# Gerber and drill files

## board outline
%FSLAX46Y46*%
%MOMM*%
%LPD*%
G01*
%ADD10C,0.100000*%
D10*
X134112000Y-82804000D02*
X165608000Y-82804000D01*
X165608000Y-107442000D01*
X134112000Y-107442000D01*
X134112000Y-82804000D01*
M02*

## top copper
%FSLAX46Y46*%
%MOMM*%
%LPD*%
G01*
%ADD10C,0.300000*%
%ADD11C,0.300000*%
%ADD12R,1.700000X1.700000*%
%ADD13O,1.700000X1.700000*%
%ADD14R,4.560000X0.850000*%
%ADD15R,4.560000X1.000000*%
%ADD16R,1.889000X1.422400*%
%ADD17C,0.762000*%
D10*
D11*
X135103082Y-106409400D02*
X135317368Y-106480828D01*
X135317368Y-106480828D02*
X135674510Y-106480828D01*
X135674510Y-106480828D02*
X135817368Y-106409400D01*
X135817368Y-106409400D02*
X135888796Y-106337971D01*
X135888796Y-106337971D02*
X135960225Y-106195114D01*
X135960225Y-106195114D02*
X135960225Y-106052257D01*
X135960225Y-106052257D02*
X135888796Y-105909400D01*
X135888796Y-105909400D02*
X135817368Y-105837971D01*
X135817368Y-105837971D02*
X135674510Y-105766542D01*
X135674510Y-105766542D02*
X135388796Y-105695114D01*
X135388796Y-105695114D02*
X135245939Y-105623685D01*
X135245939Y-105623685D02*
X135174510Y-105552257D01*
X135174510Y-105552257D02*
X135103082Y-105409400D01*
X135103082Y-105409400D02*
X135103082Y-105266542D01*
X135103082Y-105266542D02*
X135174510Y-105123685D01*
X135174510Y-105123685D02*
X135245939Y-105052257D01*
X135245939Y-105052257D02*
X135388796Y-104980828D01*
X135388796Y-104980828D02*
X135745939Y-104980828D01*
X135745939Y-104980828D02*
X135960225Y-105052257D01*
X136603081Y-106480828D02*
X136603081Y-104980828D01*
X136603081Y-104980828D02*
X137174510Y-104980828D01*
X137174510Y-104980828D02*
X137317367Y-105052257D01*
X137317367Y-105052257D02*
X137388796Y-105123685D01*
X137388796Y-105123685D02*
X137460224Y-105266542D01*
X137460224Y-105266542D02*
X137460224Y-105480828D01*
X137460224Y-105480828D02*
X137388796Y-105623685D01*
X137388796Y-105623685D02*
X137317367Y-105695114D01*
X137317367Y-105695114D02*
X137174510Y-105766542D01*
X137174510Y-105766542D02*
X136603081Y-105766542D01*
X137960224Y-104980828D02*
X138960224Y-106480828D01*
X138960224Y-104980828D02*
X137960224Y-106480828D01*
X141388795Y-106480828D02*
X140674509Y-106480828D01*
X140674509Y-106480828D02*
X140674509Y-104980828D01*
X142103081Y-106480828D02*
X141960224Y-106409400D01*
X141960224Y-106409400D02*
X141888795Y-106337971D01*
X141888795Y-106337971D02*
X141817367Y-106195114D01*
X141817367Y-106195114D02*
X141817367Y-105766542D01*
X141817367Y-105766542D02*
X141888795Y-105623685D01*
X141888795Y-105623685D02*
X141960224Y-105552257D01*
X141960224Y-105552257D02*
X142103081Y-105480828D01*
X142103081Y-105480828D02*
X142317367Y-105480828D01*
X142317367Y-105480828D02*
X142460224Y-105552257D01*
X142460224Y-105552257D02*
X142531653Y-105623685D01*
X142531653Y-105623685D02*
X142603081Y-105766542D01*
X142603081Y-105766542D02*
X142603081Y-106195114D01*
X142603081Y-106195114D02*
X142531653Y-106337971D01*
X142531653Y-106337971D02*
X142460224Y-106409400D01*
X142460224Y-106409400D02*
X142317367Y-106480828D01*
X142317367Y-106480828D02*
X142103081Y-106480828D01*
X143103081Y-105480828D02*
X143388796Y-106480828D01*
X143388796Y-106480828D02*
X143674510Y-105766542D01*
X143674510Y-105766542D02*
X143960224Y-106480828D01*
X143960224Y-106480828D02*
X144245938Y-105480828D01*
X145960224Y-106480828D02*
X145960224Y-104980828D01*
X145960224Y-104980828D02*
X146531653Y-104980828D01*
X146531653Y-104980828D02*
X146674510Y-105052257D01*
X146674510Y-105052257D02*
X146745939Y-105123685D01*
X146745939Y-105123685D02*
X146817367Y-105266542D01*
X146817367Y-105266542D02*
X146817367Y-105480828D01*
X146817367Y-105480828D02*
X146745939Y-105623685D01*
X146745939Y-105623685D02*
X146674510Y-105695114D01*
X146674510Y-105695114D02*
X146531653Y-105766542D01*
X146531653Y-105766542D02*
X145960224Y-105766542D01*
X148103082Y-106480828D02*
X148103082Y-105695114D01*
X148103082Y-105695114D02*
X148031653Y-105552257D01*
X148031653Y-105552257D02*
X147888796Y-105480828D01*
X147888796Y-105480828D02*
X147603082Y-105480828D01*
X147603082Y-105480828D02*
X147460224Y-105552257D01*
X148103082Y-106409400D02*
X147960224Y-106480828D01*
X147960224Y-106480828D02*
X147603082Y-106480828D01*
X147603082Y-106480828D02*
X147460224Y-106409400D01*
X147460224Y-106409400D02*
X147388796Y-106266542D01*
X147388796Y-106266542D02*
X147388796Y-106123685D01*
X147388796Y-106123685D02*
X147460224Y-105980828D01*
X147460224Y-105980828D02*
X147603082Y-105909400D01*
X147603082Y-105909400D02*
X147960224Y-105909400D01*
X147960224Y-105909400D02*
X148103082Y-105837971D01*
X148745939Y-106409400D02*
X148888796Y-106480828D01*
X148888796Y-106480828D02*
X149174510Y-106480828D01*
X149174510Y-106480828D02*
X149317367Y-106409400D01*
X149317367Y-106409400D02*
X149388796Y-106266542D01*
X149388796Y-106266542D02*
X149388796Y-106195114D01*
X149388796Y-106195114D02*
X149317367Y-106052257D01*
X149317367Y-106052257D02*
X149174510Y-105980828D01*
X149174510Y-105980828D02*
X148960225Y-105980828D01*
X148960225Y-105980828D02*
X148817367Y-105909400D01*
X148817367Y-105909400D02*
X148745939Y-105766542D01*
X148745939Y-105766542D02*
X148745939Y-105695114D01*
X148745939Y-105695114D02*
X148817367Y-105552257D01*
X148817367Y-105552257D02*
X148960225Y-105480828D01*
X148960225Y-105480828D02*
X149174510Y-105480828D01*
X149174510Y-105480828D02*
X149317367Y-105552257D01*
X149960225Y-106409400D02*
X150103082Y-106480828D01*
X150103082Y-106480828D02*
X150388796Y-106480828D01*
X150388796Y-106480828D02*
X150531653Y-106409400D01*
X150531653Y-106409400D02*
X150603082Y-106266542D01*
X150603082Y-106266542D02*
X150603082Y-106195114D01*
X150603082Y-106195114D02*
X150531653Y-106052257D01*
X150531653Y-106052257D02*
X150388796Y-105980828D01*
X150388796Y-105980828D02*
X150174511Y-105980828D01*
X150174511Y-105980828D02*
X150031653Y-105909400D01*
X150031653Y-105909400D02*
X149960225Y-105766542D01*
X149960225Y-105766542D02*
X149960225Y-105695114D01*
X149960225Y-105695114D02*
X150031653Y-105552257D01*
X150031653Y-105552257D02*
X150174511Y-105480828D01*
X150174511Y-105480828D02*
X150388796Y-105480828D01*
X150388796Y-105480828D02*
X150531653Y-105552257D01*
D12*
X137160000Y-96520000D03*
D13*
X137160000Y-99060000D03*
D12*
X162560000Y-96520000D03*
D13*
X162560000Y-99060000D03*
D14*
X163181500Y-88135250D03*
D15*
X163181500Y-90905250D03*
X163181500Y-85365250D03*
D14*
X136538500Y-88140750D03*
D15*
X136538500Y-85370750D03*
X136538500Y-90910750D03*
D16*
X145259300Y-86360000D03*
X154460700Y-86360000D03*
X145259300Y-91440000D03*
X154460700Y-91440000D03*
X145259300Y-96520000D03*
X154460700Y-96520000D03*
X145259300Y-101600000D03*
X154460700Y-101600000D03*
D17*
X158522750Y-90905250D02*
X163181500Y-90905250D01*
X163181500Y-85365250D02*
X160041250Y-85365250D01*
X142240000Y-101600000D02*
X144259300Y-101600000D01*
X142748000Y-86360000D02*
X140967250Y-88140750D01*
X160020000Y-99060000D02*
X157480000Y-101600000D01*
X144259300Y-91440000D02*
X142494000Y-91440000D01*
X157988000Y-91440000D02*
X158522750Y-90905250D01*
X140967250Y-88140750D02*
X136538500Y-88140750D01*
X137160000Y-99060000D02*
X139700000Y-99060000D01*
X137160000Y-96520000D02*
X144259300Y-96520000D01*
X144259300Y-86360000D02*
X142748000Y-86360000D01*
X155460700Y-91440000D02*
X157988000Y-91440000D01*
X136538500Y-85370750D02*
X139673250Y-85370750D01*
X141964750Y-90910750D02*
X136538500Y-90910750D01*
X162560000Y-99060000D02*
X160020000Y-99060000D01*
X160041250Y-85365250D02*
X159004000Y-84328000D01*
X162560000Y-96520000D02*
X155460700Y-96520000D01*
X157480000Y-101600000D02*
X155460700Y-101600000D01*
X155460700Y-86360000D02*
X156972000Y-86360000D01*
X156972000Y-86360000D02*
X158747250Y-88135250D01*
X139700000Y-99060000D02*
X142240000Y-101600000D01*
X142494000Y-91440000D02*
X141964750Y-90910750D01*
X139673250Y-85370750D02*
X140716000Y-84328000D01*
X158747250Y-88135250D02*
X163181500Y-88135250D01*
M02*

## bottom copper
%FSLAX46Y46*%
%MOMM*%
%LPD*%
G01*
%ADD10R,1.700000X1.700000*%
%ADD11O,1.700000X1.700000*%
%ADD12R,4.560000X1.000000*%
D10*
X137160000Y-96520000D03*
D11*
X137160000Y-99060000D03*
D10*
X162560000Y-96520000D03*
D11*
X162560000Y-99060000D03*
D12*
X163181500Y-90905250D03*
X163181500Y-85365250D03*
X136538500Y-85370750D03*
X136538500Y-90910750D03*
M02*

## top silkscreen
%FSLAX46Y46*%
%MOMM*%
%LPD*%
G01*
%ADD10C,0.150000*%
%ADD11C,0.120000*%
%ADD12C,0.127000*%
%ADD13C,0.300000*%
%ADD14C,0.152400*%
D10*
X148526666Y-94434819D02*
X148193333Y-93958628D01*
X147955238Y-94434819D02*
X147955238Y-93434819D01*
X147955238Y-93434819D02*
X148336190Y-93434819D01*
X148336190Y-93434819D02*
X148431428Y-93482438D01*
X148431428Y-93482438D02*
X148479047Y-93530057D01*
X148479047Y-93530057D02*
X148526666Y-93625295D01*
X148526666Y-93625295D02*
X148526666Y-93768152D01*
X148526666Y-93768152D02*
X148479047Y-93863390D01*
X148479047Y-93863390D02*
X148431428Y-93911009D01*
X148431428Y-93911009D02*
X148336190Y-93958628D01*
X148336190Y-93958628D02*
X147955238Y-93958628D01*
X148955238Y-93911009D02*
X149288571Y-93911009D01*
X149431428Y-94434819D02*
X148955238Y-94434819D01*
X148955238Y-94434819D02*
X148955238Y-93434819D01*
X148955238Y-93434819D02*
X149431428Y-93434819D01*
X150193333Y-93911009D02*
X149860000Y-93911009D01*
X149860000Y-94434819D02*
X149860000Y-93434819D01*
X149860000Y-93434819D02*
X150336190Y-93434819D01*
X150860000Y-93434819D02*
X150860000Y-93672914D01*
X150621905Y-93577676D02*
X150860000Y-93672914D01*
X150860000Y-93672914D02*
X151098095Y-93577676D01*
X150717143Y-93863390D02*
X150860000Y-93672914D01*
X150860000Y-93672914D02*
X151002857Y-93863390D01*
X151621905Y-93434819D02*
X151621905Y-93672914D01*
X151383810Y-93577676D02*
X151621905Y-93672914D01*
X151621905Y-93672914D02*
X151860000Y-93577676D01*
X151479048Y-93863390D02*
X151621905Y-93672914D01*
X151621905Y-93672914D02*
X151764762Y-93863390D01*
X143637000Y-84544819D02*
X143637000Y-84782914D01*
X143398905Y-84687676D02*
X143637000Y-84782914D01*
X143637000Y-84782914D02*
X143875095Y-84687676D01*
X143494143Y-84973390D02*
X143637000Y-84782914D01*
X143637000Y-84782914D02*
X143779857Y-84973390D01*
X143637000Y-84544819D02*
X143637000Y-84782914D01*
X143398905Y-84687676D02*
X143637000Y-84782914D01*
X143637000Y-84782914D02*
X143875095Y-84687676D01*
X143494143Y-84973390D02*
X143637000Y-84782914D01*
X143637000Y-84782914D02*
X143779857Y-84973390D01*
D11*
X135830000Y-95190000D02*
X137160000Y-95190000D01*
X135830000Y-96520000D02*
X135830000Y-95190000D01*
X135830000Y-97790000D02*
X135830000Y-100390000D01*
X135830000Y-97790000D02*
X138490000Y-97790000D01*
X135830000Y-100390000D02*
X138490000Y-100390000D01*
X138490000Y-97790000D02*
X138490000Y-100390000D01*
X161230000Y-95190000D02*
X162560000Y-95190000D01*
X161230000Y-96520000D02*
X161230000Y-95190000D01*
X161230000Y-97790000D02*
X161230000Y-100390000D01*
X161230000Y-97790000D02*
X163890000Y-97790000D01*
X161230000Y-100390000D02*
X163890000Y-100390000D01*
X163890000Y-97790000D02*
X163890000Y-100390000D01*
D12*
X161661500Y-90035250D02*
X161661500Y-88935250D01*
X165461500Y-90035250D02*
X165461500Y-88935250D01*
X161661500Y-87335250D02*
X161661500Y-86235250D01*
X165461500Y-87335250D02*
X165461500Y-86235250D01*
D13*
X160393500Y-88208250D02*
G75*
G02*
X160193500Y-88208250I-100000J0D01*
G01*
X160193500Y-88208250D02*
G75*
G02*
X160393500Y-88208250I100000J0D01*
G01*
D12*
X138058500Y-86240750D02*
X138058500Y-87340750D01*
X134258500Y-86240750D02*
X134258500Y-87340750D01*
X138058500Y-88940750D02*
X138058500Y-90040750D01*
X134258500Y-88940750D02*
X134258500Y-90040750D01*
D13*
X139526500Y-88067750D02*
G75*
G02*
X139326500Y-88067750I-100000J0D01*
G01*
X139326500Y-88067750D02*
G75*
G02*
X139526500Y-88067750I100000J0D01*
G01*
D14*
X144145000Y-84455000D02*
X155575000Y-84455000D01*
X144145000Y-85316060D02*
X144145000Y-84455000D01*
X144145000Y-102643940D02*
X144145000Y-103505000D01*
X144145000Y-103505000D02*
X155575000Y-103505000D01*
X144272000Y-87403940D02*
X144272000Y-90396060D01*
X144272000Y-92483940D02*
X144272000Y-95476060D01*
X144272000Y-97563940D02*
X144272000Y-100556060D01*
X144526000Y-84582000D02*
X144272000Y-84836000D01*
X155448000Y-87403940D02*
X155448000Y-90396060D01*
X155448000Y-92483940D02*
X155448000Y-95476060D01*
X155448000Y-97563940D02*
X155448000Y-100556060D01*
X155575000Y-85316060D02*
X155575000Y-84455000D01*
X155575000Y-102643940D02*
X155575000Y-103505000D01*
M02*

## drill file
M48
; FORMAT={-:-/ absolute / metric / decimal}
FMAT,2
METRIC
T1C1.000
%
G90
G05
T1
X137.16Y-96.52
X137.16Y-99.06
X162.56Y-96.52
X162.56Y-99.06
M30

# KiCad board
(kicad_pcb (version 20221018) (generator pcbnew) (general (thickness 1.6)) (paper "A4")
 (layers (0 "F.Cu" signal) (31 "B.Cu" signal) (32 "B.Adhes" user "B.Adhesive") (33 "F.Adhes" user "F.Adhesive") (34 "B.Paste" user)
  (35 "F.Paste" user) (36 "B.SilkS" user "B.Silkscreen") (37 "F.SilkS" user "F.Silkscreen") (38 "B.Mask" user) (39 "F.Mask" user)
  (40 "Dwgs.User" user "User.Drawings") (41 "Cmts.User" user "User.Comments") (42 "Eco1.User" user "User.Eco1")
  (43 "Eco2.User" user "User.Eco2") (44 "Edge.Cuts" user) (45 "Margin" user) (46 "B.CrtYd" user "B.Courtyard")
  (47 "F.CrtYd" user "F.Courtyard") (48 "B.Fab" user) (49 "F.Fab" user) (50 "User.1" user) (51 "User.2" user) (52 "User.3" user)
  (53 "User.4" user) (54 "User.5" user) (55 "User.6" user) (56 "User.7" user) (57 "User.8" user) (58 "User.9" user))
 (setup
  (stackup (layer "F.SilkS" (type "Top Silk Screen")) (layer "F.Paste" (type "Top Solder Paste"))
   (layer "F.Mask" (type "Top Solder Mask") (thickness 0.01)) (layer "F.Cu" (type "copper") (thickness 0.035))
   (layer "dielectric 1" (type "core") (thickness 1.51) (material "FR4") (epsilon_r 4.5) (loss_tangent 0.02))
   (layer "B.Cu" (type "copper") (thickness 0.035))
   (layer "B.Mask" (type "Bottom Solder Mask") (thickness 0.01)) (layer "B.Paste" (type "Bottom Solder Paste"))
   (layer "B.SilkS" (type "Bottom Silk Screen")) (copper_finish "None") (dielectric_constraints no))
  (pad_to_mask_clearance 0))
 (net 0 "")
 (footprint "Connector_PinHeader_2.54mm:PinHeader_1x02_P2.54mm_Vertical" (layer "F.Cu") (at 137.16 96.52)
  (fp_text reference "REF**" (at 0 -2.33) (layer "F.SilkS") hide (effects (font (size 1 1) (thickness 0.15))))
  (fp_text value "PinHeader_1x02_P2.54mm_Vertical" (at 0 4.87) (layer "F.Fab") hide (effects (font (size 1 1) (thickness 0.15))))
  (fp_line (start -1.33 -1.33) (end 0 -1.33) (stroke (width 0.12) (type solid)) (layer "F.SilkS"))
  (fp_line (start -1.33 0) (end -1.33 -1.33) (stroke (width 0.12) (type solid)) (layer "F.SilkS"))
  (fp_line (start -1.33 1.27) (end -1.33 3.87) (stroke (width 0.12) (type solid)) (layer "F.SilkS"))
  (fp_line (start -1.33 1.27) (end 1.33 1.27) (stroke (width 0.12) (type solid)) (layer "F.SilkS"))
  (fp_line (start -1.33 3.87) (end 1.33 3.87) (stroke (width 0.12) (type solid)) (layer "F.SilkS"))
  (fp_line (start 1.33 1.27) (end 1.33 3.87) (stroke (width 0.12) (type solid)) (layer "F.SilkS"))
  (pad "1" thru_hole rect (at 0 0) (size 1.7 1.7) (drill 1) (layers "*.Cu" "*.Mask"))
  (pad "2" thru_hole oval (at 0 2.54) (size 1.7 1.7) (drill 1) (layers "*.Cu" "*.Mask")))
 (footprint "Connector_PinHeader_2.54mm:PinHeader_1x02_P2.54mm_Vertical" (layer "F.Cu") (at 162.56 96.52)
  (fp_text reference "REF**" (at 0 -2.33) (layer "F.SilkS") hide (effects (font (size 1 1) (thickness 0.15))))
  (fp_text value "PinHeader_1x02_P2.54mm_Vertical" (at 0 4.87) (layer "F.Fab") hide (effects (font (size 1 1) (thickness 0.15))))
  (fp_line (start -1.33 -1.33) (end 0 -1.33) (stroke (width 0.12) (type solid)) (layer "F.SilkS"))
  (fp_line (start -1.33 0) (end -1.33 -1.33) (stroke (width 0.12) (type solid)) (layer "F.SilkS"))
  (fp_line (start -1.33 1.27) (end -1.33 3.87) (stroke (width 0.12) (type solid)) (layer "F.SilkS"))
  (fp_line (start -1.33 1.27) (end 1.33 1.27) (stroke (width 0.12) (type solid)) (layer "F.SilkS"))
  (fp_line (start -1.33 3.87) (end 1.33 3.87) (stroke (width 0.12) (type solid)) (layer "F.SilkS"))
  (fp_line (start 1.33 1.27) (end 1.33 3.87) (stroke (width 0.12) (type solid)) (layer "F.SilkS"))
  (pad "1" thru_hole rect (at 0 0) (size 1.7 1.7) (drill 1) (layers "*.Cu" "*.Mask"))
  (pad "2" thru_hole oval (at 0 2.54) (size 1.7 1.7) (drill 1) (layers "*.Cu" "*.Mask")))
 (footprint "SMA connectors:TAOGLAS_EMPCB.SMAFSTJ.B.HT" (layer "F.Cu") (at 163.1815 88.13525 90)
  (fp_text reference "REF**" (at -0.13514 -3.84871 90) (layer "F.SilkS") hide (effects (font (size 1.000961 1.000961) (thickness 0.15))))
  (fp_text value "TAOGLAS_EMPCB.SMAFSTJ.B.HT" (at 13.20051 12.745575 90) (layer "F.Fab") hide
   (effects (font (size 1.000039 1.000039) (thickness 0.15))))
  (fp_line (start -1.9 -1.52) (end -0.8 -1.52) (stroke (width 0.127) (type solid)) (layer "F.SilkS"))
  (fp_line (start -1.9 2.28) (end -0.8 2.28) (stroke (width 0.127) (type solid)) (layer "F.SilkS"))
  (fp_line (start 0.8 -1.52) (end 1.9 -1.52) (stroke (width 0.127) (type solid)) (layer "F.SilkS"))
  (fp_line (start 0.8 2.28) (end 1.9 2.28) (stroke (width 0.127) (type solid)) (layer "F.SilkS"))
  (fp_circle (center -0.073 -2.888) (end 0.027 -2.888) (stroke (width 0.3) (type solid)) (fill none) (layer "F.SilkS"))
  (pad "1" smd rect (at 0 0 90) (size 0.85 4.56) (layers "F.Cu" "F.Paste" "F.Mask") (solder_mask_margin 0.102))
  (pad "SH1" smd rect (at -2.77 0 90) (size 1 4.56) (layers "F.Cu" "F.Paste" "F.Mask") (solder_mask_margin 0.102))
  (pad "SH2" smd rect (at 2.77 0 90) (size 1 4.56) (layers "F.Cu" "F.Paste" "F.Mask") (solder_mask_margin 0.102))
  (pad "SH3" smd rect (at -2.77 0 90) (size 1 4.56) (layers "B.Cu" "B.Paste" "B.Mask") (solder_mask_margin 0.102))
  (pad "SH4" smd rect (at 2.77 0 90) (size 1 4.56) (layers "B.Cu" "B.Paste" "B.Mask") (solder_mask_margin 0.102)))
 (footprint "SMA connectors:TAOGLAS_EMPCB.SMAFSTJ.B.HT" (layer "F.Cu") (at 136.5385 88.14075 -90)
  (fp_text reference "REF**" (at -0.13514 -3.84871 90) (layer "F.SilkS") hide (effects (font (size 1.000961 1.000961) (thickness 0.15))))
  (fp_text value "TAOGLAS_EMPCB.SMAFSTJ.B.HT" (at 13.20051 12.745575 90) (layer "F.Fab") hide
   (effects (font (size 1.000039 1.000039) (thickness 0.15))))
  (fp_line (start -1.9 -1.52) (end -0.8 -1.52) (stroke (width 0.127) (type solid)) (layer "F.SilkS"))
  (fp_line (start -1.9 2.28) (end -0.8 2.28) (stroke (width 0.127) (type solid)) (layer "F.SilkS"))
  (fp_line (start 0.8 -1.52) (end 1.9 -1.52) (stroke (width 0.127) (type solid)) (layer "F.SilkS"))
  (fp_line (start 0.8 2.28) (end 1.9 2.28) (stroke (width 0.127) (type solid)) (layer "F.SilkS"))
  (fp_circle (center -0.073 -2.888) (end 0.027 -2.888) (stroke (width 0.3) (type solid)) (fill none) (layer "F.SilkS"))
  (pad "1" smd rect (at 0 0 270) (size 0.85 4.56) (layers "F.Cu" "F.Paste" "F.Mask") (solder_mask_margin 0.102))
  (pad "SH1" smd rect (at -2.77 0 270) (size 1 4.56) (layers "F.Cu" "F.Paste" "F.Mask") (solder_mask_margin 0.102))
  (pad "SH2" smd rect (at 2.77 0 270) (size 1 4.56) (layers "F.Cu" "F.Paste" "F.Mask") (solder_mask_margin 0.102))
  (pad "SH3" smd rect (at -2.77 0 270) (size 1 4.56) (layers "B.Cu" "B.Paste" "B.Mask") (solder_mask_margin 0.102))
  (pad "SH4" smd rect (at 2.77 0 270) (size 1 4.56) (layers "B.Cu" "B.Paste" "B.Mask") (solder_mask_margin 0.102)))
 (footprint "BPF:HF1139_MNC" (layer "F.Cu") (at 149.86 93.98)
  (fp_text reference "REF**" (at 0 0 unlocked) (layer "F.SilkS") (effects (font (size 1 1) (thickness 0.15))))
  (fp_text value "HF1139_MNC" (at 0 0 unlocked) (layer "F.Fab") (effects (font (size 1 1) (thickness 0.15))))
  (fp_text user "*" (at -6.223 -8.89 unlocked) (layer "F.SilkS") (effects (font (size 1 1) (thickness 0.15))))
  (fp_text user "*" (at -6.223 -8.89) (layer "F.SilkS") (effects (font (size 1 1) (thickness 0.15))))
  (fp_line (start -5.715 -9.525) (end 5.715 -9.525) (stroke (width 0.1524) (type solid)) (layer "F.SilkS"))
  (fp_line (start -5.715 -8.66394) (end -5.715 -9.525) (stroke (width 0.1524) (type solid)) (layer "F.SilkS"))
  (fp_line (start -5.715 8.66394) (end -5.715 9.525) (stroke (width 0.1524) (type solid)) (layer "F.SilkS"))
  (fp_line (start -5.715 9.525) (end 5.715 9.525) (stroke (width 0.1524) (type solid)) (layer "F.SilkS"))
  (fp_line (start -5.588 -6.57606) (end -5.588 -3.58394) (stroke (width 0.1524) (type solid)) (layer "F.SilkS"))
  (fp_line (start -5.588 -1.49606) (end -5.588 1.49606) (stroke (width 0.1524) (type solid)) (layer "F.SilkS"))
  (fp_line (start -5.588 3.58394) (end -5.588 6.57606) (stroke (width 0.1524) (type solid)) (layer "F.SilkS"))
  (fp_line (start -5.334 -9.398) (end -5.588 -9.144) (stroke (width 0.1524) (type solid)) (layer "F.SilkS"))
  (fp_line (start 5.588 -6.57606) (end 5.588 -3.58394) (stroke (width 0.1524) (type solid)) (layer "F.SilkS"))
  (fp_line (start 5.588 -1.49606) (end 5.588 1.49606) (stroke (width 0.1524) (type solid)) (layer "F.SilkS"))
  (fp_line (start 5.588 3.58394) (end 5.588 6.57606) (stroke (width 0.1524) (type solid)) (layer "F.SilkS"))
  (fp_line (start 5.715 -8.66394) (end 5.715 -9.525) (stroke (width 0.1524) (type solid)) (layer "F.SilkS"))
  (fp_line (start 5.715 8.66394) (end 5.715 9.525) (stroke (width 0.1524) (type solid)) (layer "F.SilkS"))
  (pad "1" smd rect (at -4.6007 -7.62) (size 1.889 1.4224) (layers "F.Cu" "F.Paste" "F.Mask"))
  (pad "2" smd rect (at 4.6007 -7.62) (size 1.889 1.4224) (layers "F.Cu" "F.Paste" "F.Mask"))
  (pad "3" smd rect (at -4.6007 -2.54) (size 1.889 1.4224) (layers "F.Cu" "F.Paste" "F.Mask"))
  (pad "4" smd rect (at 4.6007 -2.54) (size 1.889 1.4224) (layers "F.Cu" "F.Paste" "F.Mask"))
  (pad "5" smd rect (at -4.6007 2.54) (size 1.889 1.4224) (layers "F.Cu" "F.Paste" "F.Mask"))
  (pad "6" smd rect (at 4.6007 2.54) (size 1.889 1.4224) (layers "F.Cu" "F.Paste" "F.Mask"))
  (pad "7" smd rect (at -4.6007 7.62) (size 1.889 1.4224) (layers "F.Cu" "F.Paste" "F.Mask"))
  (pad "8" smd rect (at 4.6007 7.62) (size 1.889 1.4224) (layers "F.Cu" "F.Paste" "F.Mask")))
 (gr_rect (start 134.112 82.804) (end 165.608 107.442) (stroke (width 0.1) (type default)) (fill none) (layer "Edge.Cuts"))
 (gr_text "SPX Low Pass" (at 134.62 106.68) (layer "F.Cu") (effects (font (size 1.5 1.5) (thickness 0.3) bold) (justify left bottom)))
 (segment (start 158.52275 90.90525) (end 163.1815 90.90525) (width 0.762) (layer "F.Cu") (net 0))
 (segment (start 163.1815 85.36525) (end 160.04125 85.36525) (width 0.762) (layer "F.Cu") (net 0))
 (segment (start 142.24 101.6) (end 144.2593 101.6) (width 0.762) (layer "F.Cu") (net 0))
 (segment (start 142.748 86.36) (end 140.96725 88.14075) (width 0.762) (layer "F.Cu") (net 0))
 (segment (start 160.02 99.06) (end 157.48 101.6) (width 0.762) (layer "F.Cu") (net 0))
 (segment (start 144.2593 91.44) (end 142.494 91.44) (width 0.762) (layer "F.Cu") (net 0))
 (segment (start 157.988 91.44) (end 158.52275 90.90525) (width 0.762) (layer "F.Cu") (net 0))
 (segment (start 140.96725 88.14075) (end 136.5385 88.14075) (width 0.762) (layer "F.Cu") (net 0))
 (segment (start 137.16 99.06) (end 139.7 99.06) (width 0.762) (layer "F.Cu") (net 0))
 (segment (start 137.16 96.52) (end 144.2593 96.52) (width 0.762) (layer "F.Cu") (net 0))
 (segment (start 144.2593 86.36) (end 142.748 86.36) (width 0.762) (layer "F.Cu") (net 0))
 (segment (start 155.4607 91.44) (end 157.988 91.44) (width 0.762) (layer "F.Cu") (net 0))
 (segment (start 136.5385 85.37075) (end 139.67325 85.37075) (width 0.762) (layer "F.Cu") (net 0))
 (segment (start 141.96475 90.91075) (end 136.5385 90.91075) (width 0.762) (layer "F.Cu") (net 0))
 (segment (start 162.56 99.06) (end 160.02 99.06) (width 0.762) (layer "F.Cu") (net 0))
 (segment (start 160.04125 85.36525) (end 159.004 84.328) (width 0.762) (layer "F.Cu") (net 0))
 (segment (start 162.56 96.52) (end 155.4607 96.52) (width 0.762) (layer "F.Cu") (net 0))
 (segment (start 157.48 101.6) (end 155.4607 101.6) (width 0.762) (layer "F.Cu") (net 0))
 (segment (start 155.4607 86.36) (end 156.972 86.36) (width 0.762) (layer "F.Cu") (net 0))
 (segment (start 156.972 86.36) (end 158.74725 88.13525) (width 0.762) (layer "F.Cu") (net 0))
 (segment (start 139.7 99.06) (end 142.24 101.6) (width 0.762) (layer "F.Cu") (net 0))
 (segment (start 142.494 91.44) (end 141.96475 90.91075) (width 0.762) (layer "F.Cu") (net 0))
 (segment (start 139.67325 85.37075) (end 140.716 84.328) (width 0.762) (layer "F.Cu") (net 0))
 (segment (start 158.74725 88.13525) (end 163.1815 88.13525) (width 0.762) (layer "F.Cu") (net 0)))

